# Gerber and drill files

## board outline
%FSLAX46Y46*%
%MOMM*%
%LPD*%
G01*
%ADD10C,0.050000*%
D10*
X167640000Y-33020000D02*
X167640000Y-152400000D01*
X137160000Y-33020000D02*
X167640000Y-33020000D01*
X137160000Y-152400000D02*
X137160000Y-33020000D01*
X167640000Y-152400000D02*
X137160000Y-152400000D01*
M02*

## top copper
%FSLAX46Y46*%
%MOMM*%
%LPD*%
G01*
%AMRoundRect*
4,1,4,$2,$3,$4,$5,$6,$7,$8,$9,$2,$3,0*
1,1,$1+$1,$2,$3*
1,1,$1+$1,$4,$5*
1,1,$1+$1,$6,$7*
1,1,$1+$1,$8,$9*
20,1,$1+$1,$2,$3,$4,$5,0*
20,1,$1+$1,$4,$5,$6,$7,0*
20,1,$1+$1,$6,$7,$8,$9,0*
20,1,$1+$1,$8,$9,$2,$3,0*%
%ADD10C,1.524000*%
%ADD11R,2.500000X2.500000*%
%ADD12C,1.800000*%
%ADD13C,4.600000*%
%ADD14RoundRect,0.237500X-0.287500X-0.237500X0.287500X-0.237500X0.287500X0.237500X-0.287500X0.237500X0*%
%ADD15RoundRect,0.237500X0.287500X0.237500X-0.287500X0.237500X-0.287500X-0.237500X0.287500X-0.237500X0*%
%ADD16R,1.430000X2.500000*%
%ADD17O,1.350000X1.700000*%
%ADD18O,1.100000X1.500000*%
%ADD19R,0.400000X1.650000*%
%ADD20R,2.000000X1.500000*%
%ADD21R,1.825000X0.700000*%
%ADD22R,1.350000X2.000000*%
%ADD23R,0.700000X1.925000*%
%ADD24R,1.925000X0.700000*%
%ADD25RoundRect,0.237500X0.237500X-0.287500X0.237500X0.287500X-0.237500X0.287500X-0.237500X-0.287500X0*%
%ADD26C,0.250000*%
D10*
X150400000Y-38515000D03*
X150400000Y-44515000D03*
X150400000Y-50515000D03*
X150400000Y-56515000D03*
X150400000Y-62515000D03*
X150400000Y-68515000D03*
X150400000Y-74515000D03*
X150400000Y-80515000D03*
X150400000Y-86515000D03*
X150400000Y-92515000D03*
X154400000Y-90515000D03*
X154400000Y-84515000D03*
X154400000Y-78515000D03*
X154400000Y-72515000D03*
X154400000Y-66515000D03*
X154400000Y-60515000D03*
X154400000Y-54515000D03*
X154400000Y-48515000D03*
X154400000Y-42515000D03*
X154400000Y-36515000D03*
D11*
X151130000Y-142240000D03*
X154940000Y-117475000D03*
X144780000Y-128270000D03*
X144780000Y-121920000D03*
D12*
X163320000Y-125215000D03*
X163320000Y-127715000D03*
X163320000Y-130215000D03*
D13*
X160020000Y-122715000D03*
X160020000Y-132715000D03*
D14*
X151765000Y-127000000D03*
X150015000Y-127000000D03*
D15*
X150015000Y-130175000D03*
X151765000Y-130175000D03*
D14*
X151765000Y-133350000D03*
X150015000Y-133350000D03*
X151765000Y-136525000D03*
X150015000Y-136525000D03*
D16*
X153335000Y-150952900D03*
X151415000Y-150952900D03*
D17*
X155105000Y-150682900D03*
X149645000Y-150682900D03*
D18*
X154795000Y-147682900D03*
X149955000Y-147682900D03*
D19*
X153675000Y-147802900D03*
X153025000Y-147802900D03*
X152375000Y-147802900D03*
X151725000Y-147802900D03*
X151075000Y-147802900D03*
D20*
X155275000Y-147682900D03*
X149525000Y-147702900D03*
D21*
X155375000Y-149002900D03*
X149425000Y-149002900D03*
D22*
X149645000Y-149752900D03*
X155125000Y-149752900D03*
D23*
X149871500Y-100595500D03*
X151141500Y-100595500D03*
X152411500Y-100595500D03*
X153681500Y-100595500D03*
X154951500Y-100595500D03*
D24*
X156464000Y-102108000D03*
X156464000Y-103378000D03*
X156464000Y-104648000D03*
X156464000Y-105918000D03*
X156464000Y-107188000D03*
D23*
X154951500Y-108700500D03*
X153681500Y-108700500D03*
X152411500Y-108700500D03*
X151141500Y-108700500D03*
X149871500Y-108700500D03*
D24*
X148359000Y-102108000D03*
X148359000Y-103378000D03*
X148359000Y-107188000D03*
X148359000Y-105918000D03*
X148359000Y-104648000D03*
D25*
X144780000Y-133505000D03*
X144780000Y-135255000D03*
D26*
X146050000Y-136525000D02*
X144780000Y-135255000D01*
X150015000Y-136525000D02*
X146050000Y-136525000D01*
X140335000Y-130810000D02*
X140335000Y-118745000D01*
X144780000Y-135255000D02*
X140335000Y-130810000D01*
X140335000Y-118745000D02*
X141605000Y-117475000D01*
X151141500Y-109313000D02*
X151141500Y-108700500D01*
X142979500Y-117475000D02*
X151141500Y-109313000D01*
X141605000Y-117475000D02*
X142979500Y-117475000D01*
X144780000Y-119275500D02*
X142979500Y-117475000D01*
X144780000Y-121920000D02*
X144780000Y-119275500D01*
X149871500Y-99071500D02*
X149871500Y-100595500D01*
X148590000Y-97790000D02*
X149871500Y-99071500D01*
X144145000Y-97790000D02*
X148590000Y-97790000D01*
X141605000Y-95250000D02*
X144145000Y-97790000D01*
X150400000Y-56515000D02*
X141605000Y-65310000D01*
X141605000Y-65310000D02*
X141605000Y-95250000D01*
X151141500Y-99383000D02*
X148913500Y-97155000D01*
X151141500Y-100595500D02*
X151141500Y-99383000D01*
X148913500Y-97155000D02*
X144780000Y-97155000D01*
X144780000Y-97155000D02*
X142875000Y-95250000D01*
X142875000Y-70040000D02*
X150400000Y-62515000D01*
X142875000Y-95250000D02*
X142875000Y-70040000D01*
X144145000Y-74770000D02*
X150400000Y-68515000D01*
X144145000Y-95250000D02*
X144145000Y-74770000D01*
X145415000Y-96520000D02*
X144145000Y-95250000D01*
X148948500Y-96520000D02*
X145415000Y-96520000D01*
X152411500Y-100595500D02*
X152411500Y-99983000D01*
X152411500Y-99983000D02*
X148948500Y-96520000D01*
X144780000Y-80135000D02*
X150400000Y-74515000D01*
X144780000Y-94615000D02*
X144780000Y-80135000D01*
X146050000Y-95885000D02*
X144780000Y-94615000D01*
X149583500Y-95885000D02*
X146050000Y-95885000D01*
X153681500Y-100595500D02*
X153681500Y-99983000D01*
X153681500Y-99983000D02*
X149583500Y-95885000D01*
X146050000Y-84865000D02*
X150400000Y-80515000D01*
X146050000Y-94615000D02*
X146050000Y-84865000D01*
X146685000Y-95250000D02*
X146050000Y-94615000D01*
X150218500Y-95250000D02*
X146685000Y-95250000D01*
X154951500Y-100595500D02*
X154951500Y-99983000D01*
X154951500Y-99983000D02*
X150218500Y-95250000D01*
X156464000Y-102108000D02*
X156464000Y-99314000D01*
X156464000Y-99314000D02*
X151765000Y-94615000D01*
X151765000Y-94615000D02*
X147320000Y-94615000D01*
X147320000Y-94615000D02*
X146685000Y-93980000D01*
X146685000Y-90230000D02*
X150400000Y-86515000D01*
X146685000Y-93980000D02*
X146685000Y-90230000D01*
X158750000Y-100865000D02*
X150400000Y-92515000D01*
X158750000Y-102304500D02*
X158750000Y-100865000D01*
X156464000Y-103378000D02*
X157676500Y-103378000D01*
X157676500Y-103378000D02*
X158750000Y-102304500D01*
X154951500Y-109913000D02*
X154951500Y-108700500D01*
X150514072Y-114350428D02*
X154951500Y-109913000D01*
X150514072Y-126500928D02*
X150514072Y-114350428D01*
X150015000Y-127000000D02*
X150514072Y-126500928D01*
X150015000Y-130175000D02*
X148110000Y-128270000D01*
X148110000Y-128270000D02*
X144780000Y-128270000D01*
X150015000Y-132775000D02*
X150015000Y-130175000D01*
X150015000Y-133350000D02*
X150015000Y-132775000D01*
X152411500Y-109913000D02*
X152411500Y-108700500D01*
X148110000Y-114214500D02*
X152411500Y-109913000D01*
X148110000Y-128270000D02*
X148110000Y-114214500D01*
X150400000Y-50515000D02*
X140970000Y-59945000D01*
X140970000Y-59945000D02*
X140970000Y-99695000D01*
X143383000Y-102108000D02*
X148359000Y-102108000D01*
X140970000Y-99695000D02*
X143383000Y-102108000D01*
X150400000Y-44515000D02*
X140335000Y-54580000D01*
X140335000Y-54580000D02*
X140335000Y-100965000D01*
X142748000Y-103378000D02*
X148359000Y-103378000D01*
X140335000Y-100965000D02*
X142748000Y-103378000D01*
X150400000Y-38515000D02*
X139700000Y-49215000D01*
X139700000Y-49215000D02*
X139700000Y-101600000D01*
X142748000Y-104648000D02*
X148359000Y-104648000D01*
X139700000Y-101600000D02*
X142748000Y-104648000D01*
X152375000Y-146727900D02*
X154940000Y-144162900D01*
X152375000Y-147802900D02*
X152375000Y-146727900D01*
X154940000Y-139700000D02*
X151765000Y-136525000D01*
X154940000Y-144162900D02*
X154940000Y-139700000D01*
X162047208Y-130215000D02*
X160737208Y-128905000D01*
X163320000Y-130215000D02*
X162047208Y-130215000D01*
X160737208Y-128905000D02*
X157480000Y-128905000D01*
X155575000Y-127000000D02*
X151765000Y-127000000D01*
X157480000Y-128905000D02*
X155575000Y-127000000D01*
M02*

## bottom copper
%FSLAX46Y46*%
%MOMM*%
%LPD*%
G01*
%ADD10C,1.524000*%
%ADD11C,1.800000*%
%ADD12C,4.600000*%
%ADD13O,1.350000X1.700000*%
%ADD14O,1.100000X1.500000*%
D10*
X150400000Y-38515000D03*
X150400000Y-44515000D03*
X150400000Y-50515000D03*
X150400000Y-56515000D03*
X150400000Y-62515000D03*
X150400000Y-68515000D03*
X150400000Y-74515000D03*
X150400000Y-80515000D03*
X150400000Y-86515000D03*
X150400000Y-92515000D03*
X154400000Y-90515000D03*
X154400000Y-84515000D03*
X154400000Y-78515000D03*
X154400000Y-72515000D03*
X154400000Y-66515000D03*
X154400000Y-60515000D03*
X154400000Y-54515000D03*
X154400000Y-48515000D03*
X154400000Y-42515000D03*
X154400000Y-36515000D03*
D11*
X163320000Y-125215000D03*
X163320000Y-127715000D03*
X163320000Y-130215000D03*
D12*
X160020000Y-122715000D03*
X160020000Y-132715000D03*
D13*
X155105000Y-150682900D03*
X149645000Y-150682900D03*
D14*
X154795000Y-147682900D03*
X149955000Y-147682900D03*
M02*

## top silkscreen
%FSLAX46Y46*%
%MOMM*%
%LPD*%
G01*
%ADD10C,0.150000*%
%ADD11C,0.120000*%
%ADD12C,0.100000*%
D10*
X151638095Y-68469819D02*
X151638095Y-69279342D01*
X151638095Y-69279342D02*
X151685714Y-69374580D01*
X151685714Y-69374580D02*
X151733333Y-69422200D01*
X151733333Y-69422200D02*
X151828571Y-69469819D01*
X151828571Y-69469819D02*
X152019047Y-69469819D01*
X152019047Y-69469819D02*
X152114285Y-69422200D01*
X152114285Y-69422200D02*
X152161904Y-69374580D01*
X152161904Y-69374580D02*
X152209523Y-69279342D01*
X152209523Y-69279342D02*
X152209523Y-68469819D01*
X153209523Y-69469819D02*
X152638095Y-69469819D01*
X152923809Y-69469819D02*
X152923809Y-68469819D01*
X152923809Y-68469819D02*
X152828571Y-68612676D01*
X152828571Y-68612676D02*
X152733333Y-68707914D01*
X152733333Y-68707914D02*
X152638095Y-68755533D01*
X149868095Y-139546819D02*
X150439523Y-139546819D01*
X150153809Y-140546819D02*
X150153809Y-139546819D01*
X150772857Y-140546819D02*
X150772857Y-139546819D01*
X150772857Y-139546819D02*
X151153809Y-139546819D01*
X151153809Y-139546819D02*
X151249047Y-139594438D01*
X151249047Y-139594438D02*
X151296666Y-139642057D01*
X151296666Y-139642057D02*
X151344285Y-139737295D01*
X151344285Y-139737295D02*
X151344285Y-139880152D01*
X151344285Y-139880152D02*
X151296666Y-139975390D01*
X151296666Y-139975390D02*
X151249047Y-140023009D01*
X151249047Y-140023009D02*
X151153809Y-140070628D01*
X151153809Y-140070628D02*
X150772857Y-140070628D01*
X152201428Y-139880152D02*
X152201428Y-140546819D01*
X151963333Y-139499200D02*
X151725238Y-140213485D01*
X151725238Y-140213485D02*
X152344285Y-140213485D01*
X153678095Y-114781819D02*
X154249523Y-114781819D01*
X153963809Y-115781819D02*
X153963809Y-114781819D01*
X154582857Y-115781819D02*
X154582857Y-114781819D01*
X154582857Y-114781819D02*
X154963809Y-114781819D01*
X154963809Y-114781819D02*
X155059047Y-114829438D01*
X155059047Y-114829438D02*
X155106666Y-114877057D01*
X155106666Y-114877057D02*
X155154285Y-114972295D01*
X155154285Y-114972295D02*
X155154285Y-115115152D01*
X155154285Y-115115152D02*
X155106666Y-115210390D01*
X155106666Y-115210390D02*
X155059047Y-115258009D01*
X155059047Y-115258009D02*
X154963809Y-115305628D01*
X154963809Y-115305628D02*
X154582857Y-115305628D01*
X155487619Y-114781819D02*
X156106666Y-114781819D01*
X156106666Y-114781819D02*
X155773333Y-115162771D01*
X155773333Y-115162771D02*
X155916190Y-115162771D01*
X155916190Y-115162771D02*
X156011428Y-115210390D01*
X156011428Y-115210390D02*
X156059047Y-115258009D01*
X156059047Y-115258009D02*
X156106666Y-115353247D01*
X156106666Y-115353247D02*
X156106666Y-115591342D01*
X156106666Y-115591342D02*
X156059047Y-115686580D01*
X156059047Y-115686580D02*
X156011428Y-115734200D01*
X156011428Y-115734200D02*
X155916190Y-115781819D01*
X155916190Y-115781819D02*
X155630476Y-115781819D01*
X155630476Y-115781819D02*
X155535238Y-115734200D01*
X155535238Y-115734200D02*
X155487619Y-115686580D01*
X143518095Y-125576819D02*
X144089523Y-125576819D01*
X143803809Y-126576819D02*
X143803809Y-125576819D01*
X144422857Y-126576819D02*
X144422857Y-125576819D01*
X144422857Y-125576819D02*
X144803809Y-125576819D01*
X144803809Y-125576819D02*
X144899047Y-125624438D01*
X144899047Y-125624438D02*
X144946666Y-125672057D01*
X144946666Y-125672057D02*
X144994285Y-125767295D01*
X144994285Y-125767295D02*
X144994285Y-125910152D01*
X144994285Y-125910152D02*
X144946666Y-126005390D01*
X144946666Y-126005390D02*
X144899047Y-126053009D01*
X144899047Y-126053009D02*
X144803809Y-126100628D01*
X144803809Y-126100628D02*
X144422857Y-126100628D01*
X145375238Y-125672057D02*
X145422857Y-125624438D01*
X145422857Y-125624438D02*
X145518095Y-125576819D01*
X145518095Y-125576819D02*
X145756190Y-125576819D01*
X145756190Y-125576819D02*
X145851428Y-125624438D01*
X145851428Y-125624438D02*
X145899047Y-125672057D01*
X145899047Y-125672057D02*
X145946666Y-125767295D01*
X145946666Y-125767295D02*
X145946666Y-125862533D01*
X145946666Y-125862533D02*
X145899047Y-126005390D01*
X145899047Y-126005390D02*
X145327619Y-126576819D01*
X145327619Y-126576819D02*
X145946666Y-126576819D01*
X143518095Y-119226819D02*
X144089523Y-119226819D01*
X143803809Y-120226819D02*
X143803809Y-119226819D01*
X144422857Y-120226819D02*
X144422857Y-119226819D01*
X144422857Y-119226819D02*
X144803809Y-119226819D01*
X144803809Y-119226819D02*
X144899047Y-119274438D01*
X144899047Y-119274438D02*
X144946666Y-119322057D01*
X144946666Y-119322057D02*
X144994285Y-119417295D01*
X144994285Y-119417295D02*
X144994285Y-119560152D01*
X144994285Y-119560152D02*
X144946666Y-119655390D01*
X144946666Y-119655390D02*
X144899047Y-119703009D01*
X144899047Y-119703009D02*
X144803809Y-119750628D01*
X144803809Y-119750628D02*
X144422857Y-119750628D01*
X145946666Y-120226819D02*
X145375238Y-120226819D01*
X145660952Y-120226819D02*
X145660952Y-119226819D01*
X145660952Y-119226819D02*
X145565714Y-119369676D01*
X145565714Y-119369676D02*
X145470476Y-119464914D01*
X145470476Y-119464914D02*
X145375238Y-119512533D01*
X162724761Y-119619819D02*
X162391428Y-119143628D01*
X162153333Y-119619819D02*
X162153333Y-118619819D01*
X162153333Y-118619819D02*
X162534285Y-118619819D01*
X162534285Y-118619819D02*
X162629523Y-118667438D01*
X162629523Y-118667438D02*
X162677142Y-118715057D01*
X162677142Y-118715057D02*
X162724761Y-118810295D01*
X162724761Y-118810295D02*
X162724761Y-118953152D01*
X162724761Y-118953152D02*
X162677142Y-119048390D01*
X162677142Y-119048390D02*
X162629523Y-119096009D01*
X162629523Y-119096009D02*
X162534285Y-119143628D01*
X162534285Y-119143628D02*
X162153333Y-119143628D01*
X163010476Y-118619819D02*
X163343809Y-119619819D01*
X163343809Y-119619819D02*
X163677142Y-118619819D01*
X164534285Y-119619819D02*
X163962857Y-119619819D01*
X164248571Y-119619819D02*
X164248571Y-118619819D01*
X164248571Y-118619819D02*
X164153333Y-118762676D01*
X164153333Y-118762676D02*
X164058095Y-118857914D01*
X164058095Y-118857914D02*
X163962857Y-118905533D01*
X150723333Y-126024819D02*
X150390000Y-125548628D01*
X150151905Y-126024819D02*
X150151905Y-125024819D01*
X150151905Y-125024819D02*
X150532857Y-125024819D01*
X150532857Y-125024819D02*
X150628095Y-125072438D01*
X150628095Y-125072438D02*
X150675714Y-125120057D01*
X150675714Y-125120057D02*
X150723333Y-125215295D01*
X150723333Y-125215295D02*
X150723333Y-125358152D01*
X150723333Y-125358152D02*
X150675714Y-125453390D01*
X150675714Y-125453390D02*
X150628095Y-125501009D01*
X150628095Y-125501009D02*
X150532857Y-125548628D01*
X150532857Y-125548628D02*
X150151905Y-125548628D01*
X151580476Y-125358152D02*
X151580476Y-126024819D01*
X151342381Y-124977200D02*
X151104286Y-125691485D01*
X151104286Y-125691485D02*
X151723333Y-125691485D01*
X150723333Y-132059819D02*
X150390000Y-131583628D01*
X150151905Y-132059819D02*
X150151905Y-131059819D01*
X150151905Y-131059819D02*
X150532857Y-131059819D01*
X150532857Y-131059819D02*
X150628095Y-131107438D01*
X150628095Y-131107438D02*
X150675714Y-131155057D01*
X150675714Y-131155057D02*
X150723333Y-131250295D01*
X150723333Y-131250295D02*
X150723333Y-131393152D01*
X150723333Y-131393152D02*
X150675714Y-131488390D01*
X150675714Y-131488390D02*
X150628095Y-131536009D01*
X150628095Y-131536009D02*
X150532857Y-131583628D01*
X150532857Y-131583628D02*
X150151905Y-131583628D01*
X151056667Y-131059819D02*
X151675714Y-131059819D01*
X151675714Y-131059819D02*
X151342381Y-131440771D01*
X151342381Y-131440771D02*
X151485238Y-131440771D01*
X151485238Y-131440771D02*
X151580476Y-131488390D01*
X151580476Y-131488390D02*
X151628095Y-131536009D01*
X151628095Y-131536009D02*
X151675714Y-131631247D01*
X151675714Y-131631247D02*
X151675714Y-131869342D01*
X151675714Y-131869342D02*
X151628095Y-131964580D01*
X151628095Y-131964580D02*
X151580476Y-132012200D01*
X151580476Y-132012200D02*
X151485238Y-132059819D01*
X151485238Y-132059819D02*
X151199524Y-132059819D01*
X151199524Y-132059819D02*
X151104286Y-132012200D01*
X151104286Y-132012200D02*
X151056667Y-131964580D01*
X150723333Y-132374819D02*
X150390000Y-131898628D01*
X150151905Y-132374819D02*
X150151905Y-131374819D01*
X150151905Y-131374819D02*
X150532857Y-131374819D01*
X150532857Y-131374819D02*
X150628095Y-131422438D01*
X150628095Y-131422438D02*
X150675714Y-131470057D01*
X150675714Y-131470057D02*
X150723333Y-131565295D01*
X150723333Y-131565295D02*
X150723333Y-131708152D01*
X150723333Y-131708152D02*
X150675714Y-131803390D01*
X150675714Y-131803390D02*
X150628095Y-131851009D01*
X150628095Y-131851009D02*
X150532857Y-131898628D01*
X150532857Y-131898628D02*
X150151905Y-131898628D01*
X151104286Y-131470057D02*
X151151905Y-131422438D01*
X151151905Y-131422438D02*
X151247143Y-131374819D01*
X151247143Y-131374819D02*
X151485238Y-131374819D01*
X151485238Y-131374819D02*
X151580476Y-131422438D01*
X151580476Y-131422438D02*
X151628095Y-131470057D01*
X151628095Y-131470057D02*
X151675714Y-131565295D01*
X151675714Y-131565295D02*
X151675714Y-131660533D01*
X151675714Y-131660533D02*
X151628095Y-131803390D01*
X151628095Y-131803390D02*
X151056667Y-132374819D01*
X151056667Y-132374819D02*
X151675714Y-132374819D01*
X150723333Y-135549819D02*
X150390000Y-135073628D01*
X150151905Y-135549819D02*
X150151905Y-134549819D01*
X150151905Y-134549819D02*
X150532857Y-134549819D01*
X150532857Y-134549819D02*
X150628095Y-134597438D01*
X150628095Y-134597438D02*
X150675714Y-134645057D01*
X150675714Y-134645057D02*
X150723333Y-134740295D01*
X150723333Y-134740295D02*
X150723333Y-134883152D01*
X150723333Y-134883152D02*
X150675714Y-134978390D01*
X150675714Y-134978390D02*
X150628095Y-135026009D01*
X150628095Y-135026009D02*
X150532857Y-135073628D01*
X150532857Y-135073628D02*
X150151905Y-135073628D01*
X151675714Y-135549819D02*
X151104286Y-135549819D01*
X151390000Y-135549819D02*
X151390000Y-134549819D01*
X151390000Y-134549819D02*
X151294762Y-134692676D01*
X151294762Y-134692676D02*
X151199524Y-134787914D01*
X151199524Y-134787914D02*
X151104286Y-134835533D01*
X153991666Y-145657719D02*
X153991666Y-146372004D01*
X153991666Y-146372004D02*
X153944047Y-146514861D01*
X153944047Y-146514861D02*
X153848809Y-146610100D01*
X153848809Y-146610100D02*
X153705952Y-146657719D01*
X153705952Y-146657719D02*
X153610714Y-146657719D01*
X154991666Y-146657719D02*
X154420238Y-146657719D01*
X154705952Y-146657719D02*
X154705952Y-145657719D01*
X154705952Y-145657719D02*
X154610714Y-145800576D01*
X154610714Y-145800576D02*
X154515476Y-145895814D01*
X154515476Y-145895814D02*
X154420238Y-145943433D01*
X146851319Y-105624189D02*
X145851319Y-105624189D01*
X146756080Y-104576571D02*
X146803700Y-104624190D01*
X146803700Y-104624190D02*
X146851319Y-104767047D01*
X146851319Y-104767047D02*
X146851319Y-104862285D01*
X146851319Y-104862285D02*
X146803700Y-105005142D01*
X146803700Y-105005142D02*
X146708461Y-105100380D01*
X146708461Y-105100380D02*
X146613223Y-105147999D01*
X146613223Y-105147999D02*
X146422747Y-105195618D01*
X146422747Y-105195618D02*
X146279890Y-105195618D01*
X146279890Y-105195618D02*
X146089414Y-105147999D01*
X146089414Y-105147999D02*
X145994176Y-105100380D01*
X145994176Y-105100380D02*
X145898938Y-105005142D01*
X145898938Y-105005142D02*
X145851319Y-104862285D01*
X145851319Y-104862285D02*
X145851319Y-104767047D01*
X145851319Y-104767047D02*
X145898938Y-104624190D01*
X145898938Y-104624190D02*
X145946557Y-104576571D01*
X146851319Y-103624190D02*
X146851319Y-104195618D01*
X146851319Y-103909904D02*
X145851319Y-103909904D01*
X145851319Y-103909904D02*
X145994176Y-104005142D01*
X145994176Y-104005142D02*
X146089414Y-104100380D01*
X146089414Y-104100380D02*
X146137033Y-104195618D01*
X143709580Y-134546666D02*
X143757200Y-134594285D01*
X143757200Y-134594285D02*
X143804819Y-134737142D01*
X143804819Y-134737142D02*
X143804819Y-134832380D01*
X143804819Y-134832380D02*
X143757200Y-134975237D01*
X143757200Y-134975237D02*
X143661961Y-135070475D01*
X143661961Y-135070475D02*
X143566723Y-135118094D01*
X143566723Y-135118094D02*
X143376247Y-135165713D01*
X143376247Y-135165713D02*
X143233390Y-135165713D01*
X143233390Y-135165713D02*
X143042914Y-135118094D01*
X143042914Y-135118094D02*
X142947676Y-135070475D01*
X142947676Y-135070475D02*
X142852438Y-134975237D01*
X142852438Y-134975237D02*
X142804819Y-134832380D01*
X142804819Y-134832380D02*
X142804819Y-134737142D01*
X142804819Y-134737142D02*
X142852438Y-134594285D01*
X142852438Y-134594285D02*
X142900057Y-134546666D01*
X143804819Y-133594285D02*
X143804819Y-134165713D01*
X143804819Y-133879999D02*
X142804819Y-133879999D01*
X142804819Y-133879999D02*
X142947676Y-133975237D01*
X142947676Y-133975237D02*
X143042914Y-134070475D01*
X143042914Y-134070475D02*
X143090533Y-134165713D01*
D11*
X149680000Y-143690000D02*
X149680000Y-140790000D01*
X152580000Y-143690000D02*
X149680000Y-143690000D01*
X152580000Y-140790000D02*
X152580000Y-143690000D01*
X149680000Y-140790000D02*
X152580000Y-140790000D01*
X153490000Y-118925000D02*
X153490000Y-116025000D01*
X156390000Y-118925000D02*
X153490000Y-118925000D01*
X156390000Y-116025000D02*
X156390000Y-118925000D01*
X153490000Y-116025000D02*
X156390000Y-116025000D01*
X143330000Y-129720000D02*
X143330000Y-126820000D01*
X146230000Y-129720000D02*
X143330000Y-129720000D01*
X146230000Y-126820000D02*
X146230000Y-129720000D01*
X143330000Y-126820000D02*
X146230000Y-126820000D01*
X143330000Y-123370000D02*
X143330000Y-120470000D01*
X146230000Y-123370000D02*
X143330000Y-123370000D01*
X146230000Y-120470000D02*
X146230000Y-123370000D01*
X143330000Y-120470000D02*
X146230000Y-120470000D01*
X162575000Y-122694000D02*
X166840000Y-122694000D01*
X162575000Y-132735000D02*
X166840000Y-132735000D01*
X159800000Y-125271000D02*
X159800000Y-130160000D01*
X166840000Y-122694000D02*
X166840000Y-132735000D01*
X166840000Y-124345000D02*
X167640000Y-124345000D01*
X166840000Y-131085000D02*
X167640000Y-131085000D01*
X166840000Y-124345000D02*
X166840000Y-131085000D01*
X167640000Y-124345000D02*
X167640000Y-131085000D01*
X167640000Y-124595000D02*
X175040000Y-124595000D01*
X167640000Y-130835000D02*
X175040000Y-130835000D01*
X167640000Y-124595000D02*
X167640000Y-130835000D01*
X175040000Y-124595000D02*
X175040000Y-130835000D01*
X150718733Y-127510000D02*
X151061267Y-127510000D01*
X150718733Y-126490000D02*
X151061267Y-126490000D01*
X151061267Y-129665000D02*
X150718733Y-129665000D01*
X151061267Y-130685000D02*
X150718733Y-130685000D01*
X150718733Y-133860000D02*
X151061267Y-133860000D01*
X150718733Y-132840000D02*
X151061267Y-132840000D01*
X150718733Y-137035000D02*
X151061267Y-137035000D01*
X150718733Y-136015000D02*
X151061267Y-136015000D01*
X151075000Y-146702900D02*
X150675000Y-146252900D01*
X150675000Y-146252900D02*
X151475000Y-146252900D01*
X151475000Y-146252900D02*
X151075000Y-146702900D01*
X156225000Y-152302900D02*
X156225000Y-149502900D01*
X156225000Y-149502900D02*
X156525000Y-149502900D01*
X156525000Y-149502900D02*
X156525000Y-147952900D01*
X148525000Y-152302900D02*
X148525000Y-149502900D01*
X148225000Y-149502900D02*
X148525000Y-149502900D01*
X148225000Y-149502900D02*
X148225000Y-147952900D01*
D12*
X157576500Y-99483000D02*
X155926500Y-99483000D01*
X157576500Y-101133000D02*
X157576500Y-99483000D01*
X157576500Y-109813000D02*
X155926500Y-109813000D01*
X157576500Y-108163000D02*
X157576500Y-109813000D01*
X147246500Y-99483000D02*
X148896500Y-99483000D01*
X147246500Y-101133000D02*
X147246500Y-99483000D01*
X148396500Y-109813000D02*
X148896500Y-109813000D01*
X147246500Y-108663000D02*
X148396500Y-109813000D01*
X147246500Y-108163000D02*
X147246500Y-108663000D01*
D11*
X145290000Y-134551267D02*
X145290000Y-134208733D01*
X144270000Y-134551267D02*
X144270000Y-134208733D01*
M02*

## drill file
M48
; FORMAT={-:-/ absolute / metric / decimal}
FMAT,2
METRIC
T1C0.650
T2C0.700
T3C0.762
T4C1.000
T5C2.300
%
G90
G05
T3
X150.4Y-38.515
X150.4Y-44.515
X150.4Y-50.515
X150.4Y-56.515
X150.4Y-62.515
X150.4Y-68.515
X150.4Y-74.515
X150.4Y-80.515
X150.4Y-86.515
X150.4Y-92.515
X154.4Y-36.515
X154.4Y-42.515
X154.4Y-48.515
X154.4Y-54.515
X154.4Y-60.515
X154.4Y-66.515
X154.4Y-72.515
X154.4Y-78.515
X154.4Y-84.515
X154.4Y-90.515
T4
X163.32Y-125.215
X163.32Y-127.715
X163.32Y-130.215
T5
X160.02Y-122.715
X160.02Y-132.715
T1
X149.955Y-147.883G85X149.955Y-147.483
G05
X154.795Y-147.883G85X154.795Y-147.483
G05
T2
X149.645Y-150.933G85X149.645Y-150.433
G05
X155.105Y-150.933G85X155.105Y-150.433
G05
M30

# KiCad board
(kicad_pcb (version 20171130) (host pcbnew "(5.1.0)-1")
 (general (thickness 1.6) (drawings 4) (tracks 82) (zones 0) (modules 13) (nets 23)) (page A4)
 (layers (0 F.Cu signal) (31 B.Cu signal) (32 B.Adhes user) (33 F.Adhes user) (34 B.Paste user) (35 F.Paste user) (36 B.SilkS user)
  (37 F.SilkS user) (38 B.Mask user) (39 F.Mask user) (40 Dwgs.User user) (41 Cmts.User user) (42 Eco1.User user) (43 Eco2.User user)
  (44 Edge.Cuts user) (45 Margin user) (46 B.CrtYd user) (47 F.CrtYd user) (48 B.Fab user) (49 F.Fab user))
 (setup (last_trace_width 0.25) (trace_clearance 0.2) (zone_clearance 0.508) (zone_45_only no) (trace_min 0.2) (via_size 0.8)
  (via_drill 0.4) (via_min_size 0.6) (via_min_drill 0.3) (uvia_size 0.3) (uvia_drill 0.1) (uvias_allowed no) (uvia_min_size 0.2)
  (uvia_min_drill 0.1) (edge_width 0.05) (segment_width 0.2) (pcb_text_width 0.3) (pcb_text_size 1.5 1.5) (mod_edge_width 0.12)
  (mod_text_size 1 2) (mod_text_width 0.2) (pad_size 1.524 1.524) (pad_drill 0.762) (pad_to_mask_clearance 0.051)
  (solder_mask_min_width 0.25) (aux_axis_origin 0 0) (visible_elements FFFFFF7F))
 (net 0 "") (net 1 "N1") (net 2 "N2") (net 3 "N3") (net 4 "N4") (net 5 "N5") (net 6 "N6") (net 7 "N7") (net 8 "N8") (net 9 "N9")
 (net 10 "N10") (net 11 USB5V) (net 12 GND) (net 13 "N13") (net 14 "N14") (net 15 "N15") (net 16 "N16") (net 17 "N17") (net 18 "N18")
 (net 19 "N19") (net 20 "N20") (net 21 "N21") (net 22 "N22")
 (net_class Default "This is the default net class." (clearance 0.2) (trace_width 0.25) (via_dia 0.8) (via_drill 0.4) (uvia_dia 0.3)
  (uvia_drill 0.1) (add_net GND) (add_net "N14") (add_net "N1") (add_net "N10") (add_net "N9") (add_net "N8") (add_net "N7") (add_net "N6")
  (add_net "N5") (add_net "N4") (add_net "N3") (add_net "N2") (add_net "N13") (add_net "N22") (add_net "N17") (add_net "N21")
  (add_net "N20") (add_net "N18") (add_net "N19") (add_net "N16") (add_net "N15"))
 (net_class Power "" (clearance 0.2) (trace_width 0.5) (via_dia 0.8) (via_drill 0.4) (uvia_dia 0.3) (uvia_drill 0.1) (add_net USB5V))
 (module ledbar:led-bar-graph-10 (layer F.Cu) (at 152.4 68.515)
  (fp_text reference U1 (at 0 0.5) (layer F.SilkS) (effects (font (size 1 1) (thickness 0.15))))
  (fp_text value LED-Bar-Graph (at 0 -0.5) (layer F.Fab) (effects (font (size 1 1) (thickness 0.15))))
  (pad 1 thru_hole circle (at -2 -30) (size 1.524 1.524) (drill 0.762) (layers *.Cu *.Mask) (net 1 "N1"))
  (pad 2 thru_hole circle (at -2 -24) (size 1.524 1.524) (drill 0.762) (layers *.Cu *.Mask) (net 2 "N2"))
  (pad 3 thru_hole circle (at -2 -18) (size 1.524 1.524) (drill 0.762) (layers *.Cu *.Mask) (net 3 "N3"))
  (pad 4 thru_hole circle (at -2 -12) (size 1.524 1.524) (drill 0.762) (layers *.Cu *.Mask) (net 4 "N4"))
  (pad 5 thru_hole circle (at -2 -6) (size 1.524 1.524) (drill 0.762) (layers *.Cu *.Mask) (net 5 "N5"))
  (pad 6 thru_hole circle (at -2 0) (size 1.524 1.524) (drill 0.762) (layers *.Cu *.Mask) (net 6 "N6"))
  (pad 7 thru_hole circle (at -2 6) (size 1.524 1.524) (drill 0.762) (layers *.Cu *.Mask) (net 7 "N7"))
  (pad 8 thru_hole circle (at -2 12) (size 1.524 1.524) (drill 0.762) (layers *.Cu *.Mask) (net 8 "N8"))
  (pad 9 thru_hole circle (at -2 18) (size 1.524 1.524) (drill 0.762) (layers *.Cu *.Mask) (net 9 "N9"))
  (pad 10 thru_hole circle (at -2 24) (size 1.524 1.524) (drill 0.762) (layers *.Cu *.Mask) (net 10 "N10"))
  (pad 11 thru_hole circle (at 2 22) (size 1.524 1.524) (drill 0.762) (layers *.Cu *.Mask) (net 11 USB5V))
  (pad 12 thru_hole circle (at 2 16) (size 1.524 1.524) (drill 0.762) (layers *.Cu *.Mask) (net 11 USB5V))
  (pad 13 thru_hole circle (at 2 10) (size 1.524 1.524) (drill 0.762) (layers *.Cu *.Mask) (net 11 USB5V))
  (pad 14 thru_hole circle (at 2 4) (size 1.524 1.524) (drill 0.762) (layers *.Cu *.Mask) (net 11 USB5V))
  (pad 15 thru_hole circle (at 2 -2) (size 1.524 1.524) (drill 0.762) (layers *.Cu *.Mask) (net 11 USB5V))
  (pad 16 thru_hole circle (at 2 -8) (size 1.524 1.524) (drill 0.762) (layers *.Cu *.Mask) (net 11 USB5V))
  (pad 17 thru_hole circle (at 2 -14) (size 1.524 1.524) (drill 0.762) (layers *.Cu *.Mask) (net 11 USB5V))
  (pad 18 thru_hole circle (at 2 -20) (size 1.524 1.524) (drill 0.762) (layers *.Cu *.Mask) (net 11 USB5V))
  (pad 19 thru_hole circle (at 2 -26) (size 1.524 1.524) (drill 0.762) (layers *.Cu *.Mask) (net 11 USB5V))
  (pad 20 thru_hole circle (at 2 -32) (size 1.524 1.524) (drill 0.762) (layers *.Cu *.Mask) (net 11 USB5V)))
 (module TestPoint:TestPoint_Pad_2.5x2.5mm (layer F.Cu) (at 151.13 142.24)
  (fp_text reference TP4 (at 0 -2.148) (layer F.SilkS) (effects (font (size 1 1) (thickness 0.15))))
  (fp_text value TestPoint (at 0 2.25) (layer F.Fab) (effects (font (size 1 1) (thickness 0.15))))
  (fp_line (start -1.45 1.45) (end -1.45 -1.45) (layer F.SilkS) (width 0.12))
  (fp_line (start 1.45 1.45) (end -1.45 1.45) (layer F.SilkS) (width 0.12))
  (fp_line (start 1.45 -1.45) (end 1.45 1.45) (layer F.SilkS) (width 0.12))
  (fp_line (start -1.45 -1.45) (end 1.45 -1.45) (layer F.SilkS) (width 0.12))
  (pad 1 smd rect (at 0 0) (size 2.5 2.5) (layers F.Cu F.Mask) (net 11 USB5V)))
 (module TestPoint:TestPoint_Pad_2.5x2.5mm (layer F.Cu) (at 154.94 117.475)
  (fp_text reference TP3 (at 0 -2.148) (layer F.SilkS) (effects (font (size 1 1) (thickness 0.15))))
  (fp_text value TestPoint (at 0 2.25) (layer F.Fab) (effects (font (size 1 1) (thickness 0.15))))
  (fp_line (start -1.45 1.45) (end -1.45 -1.45) (layer F.SilkS) (width 0.12))
  (fp_line (start 1.45 1.45) (end -1.45 1.45) (layer F.SilkS) (width 0.12))
  (fp_line (start 1.45 -1.45) (end 1.45 1.45) (layer F.SilkS) (width 0.12))
  (fp_line (start -1.45 -1.45) (end 1.45 -1.45) (layer F.SilkS) (width 0.12))
  (pad 1 smd rect (at 0 0) (size 2.5 2.5) (layers F.Cu F.Mask) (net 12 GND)))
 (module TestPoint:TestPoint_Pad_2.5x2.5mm (layer F.Cu) (at 144.78 128.27)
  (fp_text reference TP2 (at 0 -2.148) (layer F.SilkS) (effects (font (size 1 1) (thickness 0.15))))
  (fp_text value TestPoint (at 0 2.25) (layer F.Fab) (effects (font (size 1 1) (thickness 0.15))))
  (fp_line (start -1.45 1.45) (end -1.45 -1.45) (layer F.SilkS) (width 0.12))
  (fp_line (start 1.45 1.45) (end -1.45 1.45) (layer F.SilkS) (width 0.12))
  (fp_line (start 1.45 -1.45) (end 1.45 1.45) (layer F.SilkS) (width 0.12))
  (fp_line (start -1.45 -1.45) (end 1.45 -1.45) (layer F.SilkS) (width 0.12))
  (pad 1 smd rect (at 0 0) (size 2.5 2.5) (layers F.Cu F.Mask) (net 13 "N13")))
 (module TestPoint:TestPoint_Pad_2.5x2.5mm (layer F.Cu) (at 144.78 121.92)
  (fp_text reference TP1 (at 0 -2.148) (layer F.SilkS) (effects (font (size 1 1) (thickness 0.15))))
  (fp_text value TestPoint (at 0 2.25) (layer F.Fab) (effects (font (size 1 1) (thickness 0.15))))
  (fp_line (start -1.45 1.45) (end -1.45 -1.45) (layer F.SilkS) (width 0.12))
  (fp_line (start 1.45 1.45) (end -1.45 1.45) (layer F.SilkS) (width 0.12))
  (fp_line (start 1.45 -1.45) (end 1.45 1.45) (layer F.SilkS) (width 0.12))
  (fp_line (start -1.45 -1.45) (end 1.45 -1.45) (layer F.SilkS) (width 0.12))
  (pad 1 smd rect (at 0 0) (size 2.5 2.5) (layers F.Cu F.Mask) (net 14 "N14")))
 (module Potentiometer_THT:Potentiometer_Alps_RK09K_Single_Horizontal (layer F.Cu) (at 163.32 130.215)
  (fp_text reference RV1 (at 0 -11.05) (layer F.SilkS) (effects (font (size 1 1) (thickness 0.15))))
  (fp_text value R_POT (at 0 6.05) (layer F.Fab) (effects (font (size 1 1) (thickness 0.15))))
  (fp_line (start -0.745 -7.521) (end 3.52 -7.521) (layer F.SilkS) (width 0.12))
  (fp_line (start -0.745 2.52) (end 3.52 2.52) (layer F.SilkS) (width 0.12))
  (fp_line (start -3.52 -4.944) (end -3.52 -0.055) (layer F.SilkS) (width 0.12))
  (fp_line (start 3.52 -7.521) (end 3.52 2.52) (layer F.SilkS) (width 0.12))
  (fp_line (start 3.52 -5.87) (end 4.32 -5.87) (layer F.SilkS) (width 0.12))
  (fp_line (start 3.52 0.87) (end 4.32 0.87) (layer F.SilkS) (width 0.12))
  (fp_line (start 3.52 -5.87) (end 3.52 0.87) (layer F.SilkS) (width 0.12))
  (fp_line (start 4.32 -5.87) (end 4.32 0.87) (layer F.SilkS) (width 0.12))
  (fp_line (start 4.32 -5.62) (end 11.72 -5.62) (layer F.SilkS) (width 0.12))
  (fp_line (start 4.32 0.62) (end 11.72 0.62) (layer F.SilkS) (width 0.12))
  (fp_line (start 4.32 -5.62) (end 4.32 0.62) (layer F.SilkS) (width 0.12))
  (fp_line (start 11.72 -5.62) (end 11.72 0.62) (layer F.SilkS) (width 0.12))
  (pad 3 thru_hole circle (at 0 -5) (size 1.8 1.8) (drill 1) (layers *.Cu *.Mask) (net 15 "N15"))
  (pad 2 thru_hole circle (at 0 -2.5) (size 1.8 1.8) (drill 1) (layers *.Cu *.Mask) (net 12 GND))
  (pad 1 thru_hole circle (at 0 0) (size 1.8 1.8) (drill 1) (layers *.Cu *.Mask) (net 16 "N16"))
  (pad "" thru_hole circle (at -3.3 -7.5) (size 4.6 4.6) (drill 2.3) (layers *.Cu *.Mask))
  (pad "" thru_hole circle (at -3.3 2.5) (size 4.6 4.6) (drill 2.3) (layers *.Cu *.Mask)))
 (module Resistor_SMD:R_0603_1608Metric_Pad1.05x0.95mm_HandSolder (layer F.Cu) (at 150.89 127)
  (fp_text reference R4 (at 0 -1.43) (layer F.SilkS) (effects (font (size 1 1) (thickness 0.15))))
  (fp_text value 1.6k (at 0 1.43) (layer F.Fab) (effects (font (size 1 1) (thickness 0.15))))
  (fp_line (start -0.171267 0.51) (end 0.171267 0.51) (layer F.SilkS) (width 0.12))
  (fp_line (start -0.171267 -0.51) (end 0.171267 -0.51) (layer F.SilkS) (width 0.12))
  (pad 2 smd roundrect (at 0.875 0) (size 1.05 0.95) (layers F.Cu F.Paste F.Mask) (roundrect_rratio 0.25) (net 16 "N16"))
  (pad 1 smd roundrect (at -0.875 0) (size 1.05 0.95) (layers F.Cu F.Paste F.Mask) (roundrect_rratio 0.25) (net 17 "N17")))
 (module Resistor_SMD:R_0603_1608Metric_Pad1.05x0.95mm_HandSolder (layer F.Cu) (at 150.89 130.175 180)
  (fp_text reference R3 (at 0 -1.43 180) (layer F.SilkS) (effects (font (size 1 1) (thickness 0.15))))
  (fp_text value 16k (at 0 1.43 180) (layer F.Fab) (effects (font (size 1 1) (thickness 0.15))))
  (fp_line (start -0.171267 0.51) (end 0.171267 0.51) (layer F.SilkS) (width 0.12))
  (fp_line (start -0.171267 -0.51) (end 0.171267 -0.51) (layer F.SilkS) (width 0.12))
  (pad 2 smd roundrect (at 0.875 0 180) (size 1.05 0.95) (layers F.Cu F.Paste F.Mask) (roundrect_rratio 0.25) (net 13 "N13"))
  (pad 1 smd roundrect (at -0.875 0 180) (size 1.05 0.95) (layers F.Cu F.Paste F.Mask) (roundrect_rratio 0.25) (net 12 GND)))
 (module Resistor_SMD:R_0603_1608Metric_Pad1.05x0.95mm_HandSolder (layer F.Cu) (at 150.89 133.35)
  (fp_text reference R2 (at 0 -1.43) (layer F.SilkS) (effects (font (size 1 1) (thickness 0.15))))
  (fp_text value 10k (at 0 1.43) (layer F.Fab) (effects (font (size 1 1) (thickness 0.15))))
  (fp_line (start -0.171267 0.51) (end 0.171267 0.51) (layer F.SilkS) (width 0.12))
  (fp_line (start -0.171267 -0.51) (end 0.171267 -0.51) (layer F.SilkS) (width 0.12))
  (pad 2 smd roundrect (at 0.875 0) (size 1.05 0.95) (layers F.Cu F.Paste F.Mask) (roundrect_rratio 0.25) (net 11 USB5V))
  (pad 1 smd roundrect (at -0.875 0) (size 1.05 0.95) (layers F.Cu F.Paste F.Mask) (roundrect_rratio 0.25) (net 13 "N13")))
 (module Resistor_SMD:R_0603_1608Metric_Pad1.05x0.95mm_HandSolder (layer F.Cu) (at 150.89 136.525)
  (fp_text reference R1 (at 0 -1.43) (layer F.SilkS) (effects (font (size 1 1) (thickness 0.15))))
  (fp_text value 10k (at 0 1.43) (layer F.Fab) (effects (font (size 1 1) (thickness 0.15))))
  (fp_line (start -0.171267 0.51) (end 0.171267 0.51) (layer F.SilkS) (width 0.12))
  (fp_line (start -0.171267 -0.51) (end 0.171267 -0.51) (layer F.SilkS) (width 0.12))
  (pad 2 smd roundrect (at 0.875 0) (size 1.05 0.95) (layers F.Cu F.Paste F.Mask) (roundrect_rratio 0.25) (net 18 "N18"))
  (pad 1 smd roundrect (at -0.875 0) (size 1.05 0.95) (layers F.Cu F.Paste F.Mask) (roundrect_rratio 0.25) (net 14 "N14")))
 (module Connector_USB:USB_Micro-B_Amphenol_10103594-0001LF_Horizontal (layer F.Cu) (at 152.4 149.5679)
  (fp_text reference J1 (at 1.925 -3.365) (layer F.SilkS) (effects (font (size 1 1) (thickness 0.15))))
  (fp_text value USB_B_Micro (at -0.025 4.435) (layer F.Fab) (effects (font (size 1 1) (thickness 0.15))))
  (fp_line (start -1.325 -2.865) (end -1.725 -3.315) (layer F.SilkS) (width 0.12))
  (fp_line (start -1.725 -3.315) (end -0.925 -3.315) (layer F.SilkS) (width 0.12))
  (fp_line (start -0.925 -3.315) (end -1.325 -2.865) (layer F.SilkS) (width 0.12))
  (fp_line (start 3.825 2.735) (end 3.825 -0.065) (layer F.SilkS) (width 0.12))
  (fp_line (start 3.825 -0.065) (end 4.125 -0.065) (layer F.SilkS) (width 0.12))
  (fp_line (start 4.125 -0.065) (end 4.125 -1.615) (layer F.SilkS) (width 0.12))
  (fp_line (start -3.875 2.735) (end -3.875 -0.065) (layer F.SilkS) (width 0.12))
  (fp_line (start -4.175 -0.065) (end -3.875 -0.065) (layer F.SilkS) (width 0.12))
  (fp_line (start -4.175 -0.065) (end -4.175 -1.615) (layer F.SilkS) (width 0.12))
  (pad 6 smd rect (at 0.935 1.385 90) (size 2.5 1.43) (layers F.Cu F.Paste F.Mask) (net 12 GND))
  (pad 6 smd rect (at -0.985 1.385 90) (size 2.5 1.43) (layers F.Cu F.Paste F.Mask) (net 12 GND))
  (pad 6 thru_hole oval (at 2.705 1.115 90) (size 1.7 1.35) (drill oval 1.2 0.7) (layers *.Cu *.Mask) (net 12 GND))
  (pad 6 thru_hole oval (at -2.755 1.115 90) (size 1.7 1.35) (drill oval 1.2 0.7) (layers *.Cu *.Mask) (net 12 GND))
  (pad 6 thru_hole oval (at 2.395 -1.885 90) (size 1.5 1.1) (drill oval 1.05 0.65) (layers *.Cu *.Mask) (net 12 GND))
  (pad 6 thru_hole oval (at -2.445 -1.885 90) (size 1.5 1.1) (drill oval 1.05 0.65) (layers *.Cu *.Mask) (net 12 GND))
  (pad 5 smd rect (at 1.275 -1.765 90) (size 1.65 0.4) (layers F.Cu F.Paste F.Mask) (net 12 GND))
  (pad 4 smd rect (at 0.625 -1.765 90) (size 1.65 0.4) (layers F.Cu F.Paste F.Mask) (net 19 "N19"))
  (pad 3 smd rect (at -0.025 -1.765 90) (size 1.65 0.4) (layers F.Cu F.Paste F.Mask) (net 18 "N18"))
  (pad 2 smd rect (at -0.675 -1.765 90) (size 1.65 0.4) (layers F.Cu F.Paste F.Mask) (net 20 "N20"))
  (pad 1 smd rect (at -1.325 -1.765 90) (size 1.65 0.4) (layers F.Cu F.Paste F.Mask) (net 11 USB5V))
  (pad 6 smd rect (at 2.875 -1.885) (size 2 1.5) (layers F.Cu F.Paste F.Mask) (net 12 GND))
  (pad 6 smd rect (at -2.875 -1.865) (size 2 1.5) (layers F.Cu F.Paste F.Mask) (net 12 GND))
  (pad 6 smd rect (at 2.975 -0.565) (size 1.825 0.7) (layers F.Cu F.Paste F.Mask) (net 12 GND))
  (pad 6 smd rect (at -2.975 -0.565) (size 1.825 0.7) (layers F.Cu F.Paste F.Mask) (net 12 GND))
  (pad 6 smd rect (at -2.755 0.185) (size 1.35 2) (layers F.Cu F.Paste F.Mask) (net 12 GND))
  (pad 6 smd rect (at 2.725 0.185) (size 1.35 2) (layers F.Cu F.Paste F.Mask) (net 12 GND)))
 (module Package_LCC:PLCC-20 (layer F.Cu) (at 152.4115 104.648 90)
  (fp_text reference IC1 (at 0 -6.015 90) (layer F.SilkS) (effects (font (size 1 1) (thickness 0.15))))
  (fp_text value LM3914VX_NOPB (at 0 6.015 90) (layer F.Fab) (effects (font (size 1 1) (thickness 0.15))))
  (fp_line (start 5.165 5.165) (end 5.165 3.515) (layer F.SilkS) (width 0.1))
  (fp_line (start 3.515 5.165) (end 5.165 5.165) (layer F.SilkS) (width 0.1))
  (fp_line (start -5.165 5.165) (end -5.165 3.515) (layer F.SilkS) (width 0.1))
  (fp_line (start -3.515 5.165) (end -5.165 5.165) (layer F.SilkS) (width 0.1))
  (fp_line (start 5.165 -5.165) (end 5.165 -3.515) (layer F.SilkS) (width 0.1))
  (fp_line (start 3.515 -5.165) (end 5.165 -5.165) (layer F.SilkS) (width 0.1))
  (fp_line (start -5.165 -4.015) (end -5.165 -3.515) (layer F.SilkS) (width 0.1))
  (fp_line (start -4.015 -5.165) (end -5.165 -4.015) (layer F.SilkS) (width 0.1))
  (fp_line (start -3.515 -5.165) (end -4.015 -5.165) (layer F.SilkS) (width 0.1))
  (pad 18 smd rect (at 4.0525 -2.54 90) (size 1.925 0.7) (layers F.Cu F.Paste F.Mask) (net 4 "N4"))
  (pad 17 smd rect (at 4.0525 -1.27 90) (size 1.925 0.7) (layers F.Cu F.Paste F.Mask) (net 5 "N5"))
  (pad 16 smd rect (at 4.0525 0 90) (size 1.925 0.7) (layers F.Cu F.Paste F.Mask) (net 6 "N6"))
  (pad 15 smd rect (at 4.0525 1.27 90) (size 1.925 0.7) (layers F.Cu F.Paste F.Mask) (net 7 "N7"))
  (pad 14 smd rect (at 4.0525 2.54 90) (size 1.925 0.7) (layers F.Cu F.Paste F.Mask) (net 8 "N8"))
  (pad 13 smd rect (at 2.54 4.0525 90) (size 0.7 1.925) (layers F.Cu F.Paste F.Mask) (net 9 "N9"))
  (pad 12 smd rect (at 1.27 4.0525 90) (size 0.7 1.925) (layers F.Cu F.Paste F.Mask) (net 10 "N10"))
  (pad 11 smd rect (at 0 4.0525 90) (size 0.7 1.925) (layers F.Cu F.Paste F.Mask) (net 11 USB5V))
  (pad 10 smd rect (at -1.27 4.0525 90) (size 0.7 1.925) (layers F.Cu F.Paste F.Mask) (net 12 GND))
  (pad 9 smd rect (at -2.54 4.0525 90) (size 0.7 1.925) (layers F.Cu F.Paste F.Mask) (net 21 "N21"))
  (pad 8 smd rect (at -4.0525 2.54 90) (size 1.925 0.7) (layers F.Cu F.Paste F.Mask) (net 17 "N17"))
  (pad 7 smd rect (at -4.0525 1.27 90) (size 1.925 0.7) (layers F.Cu F.Paste F.Mask) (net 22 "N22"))
  (pad 6 smd rect (at -4.0525 0 90) (size 1.925 0.7) (layers F.Cu F.Paste F.Mask) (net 13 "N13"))
  (pad 5 smd rect (at -4.0525 -1.27 90) (size 1.925 0.7) (layers F.Cu F.Paste F.Mask) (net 14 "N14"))
  (pad 4 smd rect (at -4.0525 -2.54 90) (size 1.925 0.7) (layers F.Cu F.Paste F.Mask) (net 12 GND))
  (pad 19 smd rect (at 2.54 -4.0525 90) (size 0.7 1.925) (layers F.Cu F.Paste F.Mask) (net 3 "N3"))
  (pad 20 smd rect (at 1.27 -4.0525 90) (size 0.7 1.925) (layers F.Cu F.Paste F.Mask) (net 2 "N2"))
  (pad 3 smd rect (at -2.54 -4.0525 90) (size 0.7 1.925) (layers F.Cu F.Paste F.Mask) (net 11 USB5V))
  (pad 2 smd rect (at -1.27 -4.0525 90) (size 0.7 1.925) (layers F.Cu F.Paste F.Mask) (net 12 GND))
  (pad 1 smd rect (at 0 -4.0525 90) (size 0.7 1.925) (layers F.Cu F.Paste F.Mask) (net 1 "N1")))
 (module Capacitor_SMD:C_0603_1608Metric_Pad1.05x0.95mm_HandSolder (layer F.Cu) (at 144.78 134.38 90)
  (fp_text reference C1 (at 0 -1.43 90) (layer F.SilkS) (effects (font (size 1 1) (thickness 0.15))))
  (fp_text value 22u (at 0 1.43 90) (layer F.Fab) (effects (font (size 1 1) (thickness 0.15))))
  (fp_line (start -0.171267 0.51) (end 0.171267 0.51) (layer F.SilkS) (width 0.12))
  (fp_line (start -0.171267 -0.51) (end 0.171267 -0.51) (layer F.SilkS) (width 0.12))
  (pad 2 smd roundrect (at 0.875 0 90) (size 1.05 0.95) (layers F.Cu F.Paste F.Mask) (roundrect_rratio 0.25) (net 12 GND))
  (pad 1 smd roundrect (at -0.875 0 90) (size 1.05 0.95) (layers F.Cu F.Paste F.Mask) (roundrect_rratio 0.25) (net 14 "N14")))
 (gr_line (start 167.64 33.02) (end 167.64 152.4) (layer Edge.Cuts) (width 0.05))
 (gr_line (start 137.16 33.02) (end 167.64 33.02) (layer Edge.Cuts) (width 0.05))
 (gr_line (start 137.16 152.4) (end 137.16 33.02) (layer Edge.Cuts) (width 0.05))
 (gr_line (start 167.64 152.4) (end 137.16 152.4) (layer Edge.Cuts) (width 0.05))
 (segment (start 146.05 136.525) (end 144.78 135.255) (width 0.25) (layer F.Cu) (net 14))
 (segment (start 150.015 136.525) (end 146.05 136.525) (width 0.25) (layer F.Cu) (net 14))
 (segment (start 140.335 130.81) (end 140.335 118.745) (width 0.25) (layer F.Cu) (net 14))
 (segment (start 144.78 135.255) (end 140.335 130.81) (width 0.25) (layer F.Cu) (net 14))
 (segment (start 140.335 118.745) (end 141.605 117.475) (width 0.25) (layer F.Cu) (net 14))
 (segment (start 151.1415 109.313) (end 151.1415 108.7005) (width 0.25) (layer F.Cu) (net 14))
 (segment (start 142.9795 117.475) (end 151.1415 109.313) (width 0.25) (layer F.Cu) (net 14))
 (segment (start 141.605 117.475) (end 142.9795 117.475) (width 0.25) (layer F.Cu) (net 14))
 (segment (start 144.78 119.2755) (end 142.9795 117.475) (width 0.25) (layer F.Cu) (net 14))
 (segment (start 144.78 121.92) (end 144.78 119.2755) (width 0.25) (layer F.Cu) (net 14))
 (segment (start 149.8715 99.0715) (end 149.8715 100.5955) (width 0.25) (layer F.Cu) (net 4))
 (segment (start 148.59 97.79) (end 149.8715 99.0715) (width 0.25) (layer F.Cu) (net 4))
 (segment (start 144.145 97.79) (end 148.59 97.79) (width 0.25) (layer F.Cu) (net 4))
 (segment (start 141.605 95.25) (end 144.145 97.79) (width 0.25) (layer F.Cu) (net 4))
 (segment (start 150.4 56.515) (end 141.605 65.31) (width 0.25) (layer F.Cu) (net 4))
 (segment (start 141.605 65.31) (end 141.605 95.25) (width 0.25) (layer F.Cu) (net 4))
 (segment (start 151.1415 99.383) (end 148.9135 97.155) (width 0.25) (layer F.Cu) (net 5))
 (segment (start 151.1415 100.5955) (end 151.1415 99.383) (width 0.25) (layer F.Cu) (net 5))
 (segment (start 148.9135 97.155) (end 144.78 97.155) (width 0.25) (layer F.Cu) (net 5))
 (segment (start 144.78 97.155) (end 142.875 95.25) (width 0.25) (layer F.Cu) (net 5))
 (segment (start 142.875 70.04) (end 150.4 62.515) (width 0.25) (layer F.Cu) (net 5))
 (segment (start 142.875 95.25) (end 142.875 70.04) (width 0.25) (layer F.Cu) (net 5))
 (segment (start 144.145 74.77) (end 150.4 68.515) (width 0.25) (layer F.Cu) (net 6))
 (segment (start 144.145 95.25) (end 144.145 74.77) (width 0.25) (layer F.Cu) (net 6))
 (segment (start 145.415 96.52) (end 144.145 95.25) (width 0.25) (layer F.Cu) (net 6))
 (segment (start 148.9485 96.52) (end 145.415 96.52) (width 0.25) (layer F.Cu) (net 6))
 (segment (start 152.4115 100.5955) (end 152.4115 99.983) (width 0.25) (layer F.Cu) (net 6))
 (segment (start 152.4115 99.983) (end 148.9485 96.52) (width 0.25) (layer F.Cu) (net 6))
 (segment (start 144.78 80.135) (end 150.4 74.515) (width 0.25) (layer F.Cu) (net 7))
 (segment (start 144.78 94.615) (end 144.78 80.135) (width 0.25) (layer F.Cu) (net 7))
 (segment (start 146.05 95.885) (end 144.78 94.615) (width 0.25) (layer F.Cu) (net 7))
 (segment (start 149.5835 95.885) (end 146.05 95.885) (width 0.25) (layer F.Cu) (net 7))
 (segment (start 153.6815 100.5955) (end 153.6815 99.983) (width 0.25) (layer F.Cu) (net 7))
 (segment (start 153.6815 99.983) (end 149.5835 95.885) (width 0.25) (layer F.Cu) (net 7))
 (segment (start 146.05 84.865) (end 150.4 80.515) (width 0.25) (layer F.Cu) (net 8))
 (segment (start 146.05 94.615) (end 146.05 84.865) (width 0.25) (layer F.Cu) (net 8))
 (segment (start 146.685 95.25) (end 146.05 94.615) (width 0.25) (layer F.Cu) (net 8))
 (segment (start 150.2185 95.25) (end 146.685 95.25) (width 0.25) (layer F.Cu) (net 8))
 (segment (start 154.9515 100.5955) (end 154.9515 99.983) (width 0.25) (layer F.Cu) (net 8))
 (segment (start 154.9515 99.983) (end 150.2185 95.25) (width 0.25) (layer F.Cu) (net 8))
 (segment (start 156.464 102.108) (end 156.464 99.314) (width 0.25) (layer F.Cu) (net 9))
 (segment (start 156.464 99.314) (end 151.765 94.615) (width 0.25) (layer F.Cu) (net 9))
 (segment (start 151.765 94.615) (end 147.32 94.615) (width 0.25) (layer F.Cu) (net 9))
 (segment (start 147.32 94.615) (end 146.685 93.98) (width 0.25) (layer F.Cu) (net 9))
 (segment (start 146.685 90.23) (end 150.4 86.515) (width 0.25) (layer F.Cu) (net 9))
 (segment (start 146.685 93.98) (end 146.685 90.23) (width 0.25) (layer F.Cu) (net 9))
 (segment (start 158.75 100.865) (end 150.4 92.515) (width 0.25) (layer F.Cu) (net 10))
 (segment (start 158.75 102.3045) (end 158.75 100.865) (width 0.25) (layer F.Cu) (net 10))
 (segment (start 156.464 103.378) (end 157.6765 103.378) (width 0.25) (layer F.Cu) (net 10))
 (segment (start 157.6765 103.378) (end 158.75 102.3045) (width 0.25) (layer F.Cu) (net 10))
 (segment (start 154.9515 109.913) (end 154.9515 108.7005) (width 0.25) (layer F.Cu) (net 17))
 (segment (start 150.514072 114.350428) (end 154.9515 109.913) (width 0.25) (layer F.Cu) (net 17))
 (segment (start 150.514072 126.500928) (end 150.514072 114.350428) (width 0.25) (layer F.Cu) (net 17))
 (segment (start 150.015 127) (end 150.514072 126.500928) (width 0.25) (layer F.Cu) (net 17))
 (segment (start 150.015 130.175) (end 148.11 128.27) (width 0.25) (layer F.Cu) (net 13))
 (segment (start 148.11 128.27) (end 144.78 128.27) (width 0.25) (layer F.Cu) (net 13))
 (segment (start 150.015 132.775) (end 150.015 130.175) (width 0.25) (layer F.Cu) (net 13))
 (segment (start 150.015 133.35) (end 150.015 132.775) (width 0.25) (layer F.Cu) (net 13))
 (segment (start 152.4115 109.913) (end 152.4115 108.7005) (width 0.25) (layer F.Cu) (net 13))
 (segment (start 148.11 114.2145) (end 152.4115 109.913) (width 0.25) (layer F.Cu) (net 13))
 (segment (start 148.11 128.27) (end 148.11 114.2145) (width 0.25) (layer F.Cu) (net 13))
 (segment (start 150.4 50.515) (end 140.97 59.945) (width 0.25) (layer F.Cu) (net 3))
 (segment (start 140.97 59.945) (end 140.97 99.695) (width 0.25) (layer F.Cu) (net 3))
 (segment (start 143.383 102.108) (end 148.359 102.108) (width 0.25) (layer F.Cu) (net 3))
 (segment (start 140.97 99.695) (end 143.383 102.108) (width 0.25) (layer F.Cu) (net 3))
 (segment (start 150.4 44.515) (end 140.335 54.58) (width 0.25) (layer F.Cu) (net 2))
 (segment (start 140.335 54.58) (end 140.335 100.965) (width 0.25) (layer F.Cu) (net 2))
 (segment (start 142.748 103.378) (end 148.359 103.378) (width 0.25) (layer F.Cu) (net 2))
 (segment (start 140.335 100.965) (end 142.748 103.378) (width 0.25) (layer F.Cu) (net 2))
 (segment (start 150.4 38.515) (end 139.7 49.215) (width 0.25) (layer F.Cu) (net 1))
 (segment (start 139.7 49.215) (end 139.7 101.6) (width 0.25) (layer F.Cu) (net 1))
 (segment (start 142.748 104.648) (end 148.359 104.648) (width 0.25) (layer F.Cu) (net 1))
 (segment (start 139.7 101.6) (end 142.748 104.648) (width 0.25) (layer F.Cu) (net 1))
 (segment (start 152.375 146.7279) (end 154.94 144.1629) (width 0.25) (layer F.Cu) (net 18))
 (segment (start 152.375 147.8029) (end 152.375 146.7279) (width 0.25) (layer F.Cu) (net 18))
 (segment (start 154.94 139.7) (end 151.765 136.525) (width 0.25) (layer F.Cu) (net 18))
 (segment (start 154.94 144.1629) (end 154.94 139.7) (width 0.25) (layer F.Cu) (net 18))
 (segment (start 162.047208 130.215) (end 160.737208 128.905) (width 0.25) (layer F.Cu) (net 16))
 (segment (start 163.32 130.215) (end 162.047208 130.215) (width 0.25) (layer F.Cu) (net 16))
 (segment (start 160.737208 128.905) (end 157.48 128.905) (width 0.25) (layer F.Cu) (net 16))
 (segment (start 155.575 127) (end 151.765 127) (width 0.25) (layer F.Cu) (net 16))
 (segment (start 157.48 128.905) (end 155.575 127) (width 0.25) (layer F.Cu) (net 16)))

